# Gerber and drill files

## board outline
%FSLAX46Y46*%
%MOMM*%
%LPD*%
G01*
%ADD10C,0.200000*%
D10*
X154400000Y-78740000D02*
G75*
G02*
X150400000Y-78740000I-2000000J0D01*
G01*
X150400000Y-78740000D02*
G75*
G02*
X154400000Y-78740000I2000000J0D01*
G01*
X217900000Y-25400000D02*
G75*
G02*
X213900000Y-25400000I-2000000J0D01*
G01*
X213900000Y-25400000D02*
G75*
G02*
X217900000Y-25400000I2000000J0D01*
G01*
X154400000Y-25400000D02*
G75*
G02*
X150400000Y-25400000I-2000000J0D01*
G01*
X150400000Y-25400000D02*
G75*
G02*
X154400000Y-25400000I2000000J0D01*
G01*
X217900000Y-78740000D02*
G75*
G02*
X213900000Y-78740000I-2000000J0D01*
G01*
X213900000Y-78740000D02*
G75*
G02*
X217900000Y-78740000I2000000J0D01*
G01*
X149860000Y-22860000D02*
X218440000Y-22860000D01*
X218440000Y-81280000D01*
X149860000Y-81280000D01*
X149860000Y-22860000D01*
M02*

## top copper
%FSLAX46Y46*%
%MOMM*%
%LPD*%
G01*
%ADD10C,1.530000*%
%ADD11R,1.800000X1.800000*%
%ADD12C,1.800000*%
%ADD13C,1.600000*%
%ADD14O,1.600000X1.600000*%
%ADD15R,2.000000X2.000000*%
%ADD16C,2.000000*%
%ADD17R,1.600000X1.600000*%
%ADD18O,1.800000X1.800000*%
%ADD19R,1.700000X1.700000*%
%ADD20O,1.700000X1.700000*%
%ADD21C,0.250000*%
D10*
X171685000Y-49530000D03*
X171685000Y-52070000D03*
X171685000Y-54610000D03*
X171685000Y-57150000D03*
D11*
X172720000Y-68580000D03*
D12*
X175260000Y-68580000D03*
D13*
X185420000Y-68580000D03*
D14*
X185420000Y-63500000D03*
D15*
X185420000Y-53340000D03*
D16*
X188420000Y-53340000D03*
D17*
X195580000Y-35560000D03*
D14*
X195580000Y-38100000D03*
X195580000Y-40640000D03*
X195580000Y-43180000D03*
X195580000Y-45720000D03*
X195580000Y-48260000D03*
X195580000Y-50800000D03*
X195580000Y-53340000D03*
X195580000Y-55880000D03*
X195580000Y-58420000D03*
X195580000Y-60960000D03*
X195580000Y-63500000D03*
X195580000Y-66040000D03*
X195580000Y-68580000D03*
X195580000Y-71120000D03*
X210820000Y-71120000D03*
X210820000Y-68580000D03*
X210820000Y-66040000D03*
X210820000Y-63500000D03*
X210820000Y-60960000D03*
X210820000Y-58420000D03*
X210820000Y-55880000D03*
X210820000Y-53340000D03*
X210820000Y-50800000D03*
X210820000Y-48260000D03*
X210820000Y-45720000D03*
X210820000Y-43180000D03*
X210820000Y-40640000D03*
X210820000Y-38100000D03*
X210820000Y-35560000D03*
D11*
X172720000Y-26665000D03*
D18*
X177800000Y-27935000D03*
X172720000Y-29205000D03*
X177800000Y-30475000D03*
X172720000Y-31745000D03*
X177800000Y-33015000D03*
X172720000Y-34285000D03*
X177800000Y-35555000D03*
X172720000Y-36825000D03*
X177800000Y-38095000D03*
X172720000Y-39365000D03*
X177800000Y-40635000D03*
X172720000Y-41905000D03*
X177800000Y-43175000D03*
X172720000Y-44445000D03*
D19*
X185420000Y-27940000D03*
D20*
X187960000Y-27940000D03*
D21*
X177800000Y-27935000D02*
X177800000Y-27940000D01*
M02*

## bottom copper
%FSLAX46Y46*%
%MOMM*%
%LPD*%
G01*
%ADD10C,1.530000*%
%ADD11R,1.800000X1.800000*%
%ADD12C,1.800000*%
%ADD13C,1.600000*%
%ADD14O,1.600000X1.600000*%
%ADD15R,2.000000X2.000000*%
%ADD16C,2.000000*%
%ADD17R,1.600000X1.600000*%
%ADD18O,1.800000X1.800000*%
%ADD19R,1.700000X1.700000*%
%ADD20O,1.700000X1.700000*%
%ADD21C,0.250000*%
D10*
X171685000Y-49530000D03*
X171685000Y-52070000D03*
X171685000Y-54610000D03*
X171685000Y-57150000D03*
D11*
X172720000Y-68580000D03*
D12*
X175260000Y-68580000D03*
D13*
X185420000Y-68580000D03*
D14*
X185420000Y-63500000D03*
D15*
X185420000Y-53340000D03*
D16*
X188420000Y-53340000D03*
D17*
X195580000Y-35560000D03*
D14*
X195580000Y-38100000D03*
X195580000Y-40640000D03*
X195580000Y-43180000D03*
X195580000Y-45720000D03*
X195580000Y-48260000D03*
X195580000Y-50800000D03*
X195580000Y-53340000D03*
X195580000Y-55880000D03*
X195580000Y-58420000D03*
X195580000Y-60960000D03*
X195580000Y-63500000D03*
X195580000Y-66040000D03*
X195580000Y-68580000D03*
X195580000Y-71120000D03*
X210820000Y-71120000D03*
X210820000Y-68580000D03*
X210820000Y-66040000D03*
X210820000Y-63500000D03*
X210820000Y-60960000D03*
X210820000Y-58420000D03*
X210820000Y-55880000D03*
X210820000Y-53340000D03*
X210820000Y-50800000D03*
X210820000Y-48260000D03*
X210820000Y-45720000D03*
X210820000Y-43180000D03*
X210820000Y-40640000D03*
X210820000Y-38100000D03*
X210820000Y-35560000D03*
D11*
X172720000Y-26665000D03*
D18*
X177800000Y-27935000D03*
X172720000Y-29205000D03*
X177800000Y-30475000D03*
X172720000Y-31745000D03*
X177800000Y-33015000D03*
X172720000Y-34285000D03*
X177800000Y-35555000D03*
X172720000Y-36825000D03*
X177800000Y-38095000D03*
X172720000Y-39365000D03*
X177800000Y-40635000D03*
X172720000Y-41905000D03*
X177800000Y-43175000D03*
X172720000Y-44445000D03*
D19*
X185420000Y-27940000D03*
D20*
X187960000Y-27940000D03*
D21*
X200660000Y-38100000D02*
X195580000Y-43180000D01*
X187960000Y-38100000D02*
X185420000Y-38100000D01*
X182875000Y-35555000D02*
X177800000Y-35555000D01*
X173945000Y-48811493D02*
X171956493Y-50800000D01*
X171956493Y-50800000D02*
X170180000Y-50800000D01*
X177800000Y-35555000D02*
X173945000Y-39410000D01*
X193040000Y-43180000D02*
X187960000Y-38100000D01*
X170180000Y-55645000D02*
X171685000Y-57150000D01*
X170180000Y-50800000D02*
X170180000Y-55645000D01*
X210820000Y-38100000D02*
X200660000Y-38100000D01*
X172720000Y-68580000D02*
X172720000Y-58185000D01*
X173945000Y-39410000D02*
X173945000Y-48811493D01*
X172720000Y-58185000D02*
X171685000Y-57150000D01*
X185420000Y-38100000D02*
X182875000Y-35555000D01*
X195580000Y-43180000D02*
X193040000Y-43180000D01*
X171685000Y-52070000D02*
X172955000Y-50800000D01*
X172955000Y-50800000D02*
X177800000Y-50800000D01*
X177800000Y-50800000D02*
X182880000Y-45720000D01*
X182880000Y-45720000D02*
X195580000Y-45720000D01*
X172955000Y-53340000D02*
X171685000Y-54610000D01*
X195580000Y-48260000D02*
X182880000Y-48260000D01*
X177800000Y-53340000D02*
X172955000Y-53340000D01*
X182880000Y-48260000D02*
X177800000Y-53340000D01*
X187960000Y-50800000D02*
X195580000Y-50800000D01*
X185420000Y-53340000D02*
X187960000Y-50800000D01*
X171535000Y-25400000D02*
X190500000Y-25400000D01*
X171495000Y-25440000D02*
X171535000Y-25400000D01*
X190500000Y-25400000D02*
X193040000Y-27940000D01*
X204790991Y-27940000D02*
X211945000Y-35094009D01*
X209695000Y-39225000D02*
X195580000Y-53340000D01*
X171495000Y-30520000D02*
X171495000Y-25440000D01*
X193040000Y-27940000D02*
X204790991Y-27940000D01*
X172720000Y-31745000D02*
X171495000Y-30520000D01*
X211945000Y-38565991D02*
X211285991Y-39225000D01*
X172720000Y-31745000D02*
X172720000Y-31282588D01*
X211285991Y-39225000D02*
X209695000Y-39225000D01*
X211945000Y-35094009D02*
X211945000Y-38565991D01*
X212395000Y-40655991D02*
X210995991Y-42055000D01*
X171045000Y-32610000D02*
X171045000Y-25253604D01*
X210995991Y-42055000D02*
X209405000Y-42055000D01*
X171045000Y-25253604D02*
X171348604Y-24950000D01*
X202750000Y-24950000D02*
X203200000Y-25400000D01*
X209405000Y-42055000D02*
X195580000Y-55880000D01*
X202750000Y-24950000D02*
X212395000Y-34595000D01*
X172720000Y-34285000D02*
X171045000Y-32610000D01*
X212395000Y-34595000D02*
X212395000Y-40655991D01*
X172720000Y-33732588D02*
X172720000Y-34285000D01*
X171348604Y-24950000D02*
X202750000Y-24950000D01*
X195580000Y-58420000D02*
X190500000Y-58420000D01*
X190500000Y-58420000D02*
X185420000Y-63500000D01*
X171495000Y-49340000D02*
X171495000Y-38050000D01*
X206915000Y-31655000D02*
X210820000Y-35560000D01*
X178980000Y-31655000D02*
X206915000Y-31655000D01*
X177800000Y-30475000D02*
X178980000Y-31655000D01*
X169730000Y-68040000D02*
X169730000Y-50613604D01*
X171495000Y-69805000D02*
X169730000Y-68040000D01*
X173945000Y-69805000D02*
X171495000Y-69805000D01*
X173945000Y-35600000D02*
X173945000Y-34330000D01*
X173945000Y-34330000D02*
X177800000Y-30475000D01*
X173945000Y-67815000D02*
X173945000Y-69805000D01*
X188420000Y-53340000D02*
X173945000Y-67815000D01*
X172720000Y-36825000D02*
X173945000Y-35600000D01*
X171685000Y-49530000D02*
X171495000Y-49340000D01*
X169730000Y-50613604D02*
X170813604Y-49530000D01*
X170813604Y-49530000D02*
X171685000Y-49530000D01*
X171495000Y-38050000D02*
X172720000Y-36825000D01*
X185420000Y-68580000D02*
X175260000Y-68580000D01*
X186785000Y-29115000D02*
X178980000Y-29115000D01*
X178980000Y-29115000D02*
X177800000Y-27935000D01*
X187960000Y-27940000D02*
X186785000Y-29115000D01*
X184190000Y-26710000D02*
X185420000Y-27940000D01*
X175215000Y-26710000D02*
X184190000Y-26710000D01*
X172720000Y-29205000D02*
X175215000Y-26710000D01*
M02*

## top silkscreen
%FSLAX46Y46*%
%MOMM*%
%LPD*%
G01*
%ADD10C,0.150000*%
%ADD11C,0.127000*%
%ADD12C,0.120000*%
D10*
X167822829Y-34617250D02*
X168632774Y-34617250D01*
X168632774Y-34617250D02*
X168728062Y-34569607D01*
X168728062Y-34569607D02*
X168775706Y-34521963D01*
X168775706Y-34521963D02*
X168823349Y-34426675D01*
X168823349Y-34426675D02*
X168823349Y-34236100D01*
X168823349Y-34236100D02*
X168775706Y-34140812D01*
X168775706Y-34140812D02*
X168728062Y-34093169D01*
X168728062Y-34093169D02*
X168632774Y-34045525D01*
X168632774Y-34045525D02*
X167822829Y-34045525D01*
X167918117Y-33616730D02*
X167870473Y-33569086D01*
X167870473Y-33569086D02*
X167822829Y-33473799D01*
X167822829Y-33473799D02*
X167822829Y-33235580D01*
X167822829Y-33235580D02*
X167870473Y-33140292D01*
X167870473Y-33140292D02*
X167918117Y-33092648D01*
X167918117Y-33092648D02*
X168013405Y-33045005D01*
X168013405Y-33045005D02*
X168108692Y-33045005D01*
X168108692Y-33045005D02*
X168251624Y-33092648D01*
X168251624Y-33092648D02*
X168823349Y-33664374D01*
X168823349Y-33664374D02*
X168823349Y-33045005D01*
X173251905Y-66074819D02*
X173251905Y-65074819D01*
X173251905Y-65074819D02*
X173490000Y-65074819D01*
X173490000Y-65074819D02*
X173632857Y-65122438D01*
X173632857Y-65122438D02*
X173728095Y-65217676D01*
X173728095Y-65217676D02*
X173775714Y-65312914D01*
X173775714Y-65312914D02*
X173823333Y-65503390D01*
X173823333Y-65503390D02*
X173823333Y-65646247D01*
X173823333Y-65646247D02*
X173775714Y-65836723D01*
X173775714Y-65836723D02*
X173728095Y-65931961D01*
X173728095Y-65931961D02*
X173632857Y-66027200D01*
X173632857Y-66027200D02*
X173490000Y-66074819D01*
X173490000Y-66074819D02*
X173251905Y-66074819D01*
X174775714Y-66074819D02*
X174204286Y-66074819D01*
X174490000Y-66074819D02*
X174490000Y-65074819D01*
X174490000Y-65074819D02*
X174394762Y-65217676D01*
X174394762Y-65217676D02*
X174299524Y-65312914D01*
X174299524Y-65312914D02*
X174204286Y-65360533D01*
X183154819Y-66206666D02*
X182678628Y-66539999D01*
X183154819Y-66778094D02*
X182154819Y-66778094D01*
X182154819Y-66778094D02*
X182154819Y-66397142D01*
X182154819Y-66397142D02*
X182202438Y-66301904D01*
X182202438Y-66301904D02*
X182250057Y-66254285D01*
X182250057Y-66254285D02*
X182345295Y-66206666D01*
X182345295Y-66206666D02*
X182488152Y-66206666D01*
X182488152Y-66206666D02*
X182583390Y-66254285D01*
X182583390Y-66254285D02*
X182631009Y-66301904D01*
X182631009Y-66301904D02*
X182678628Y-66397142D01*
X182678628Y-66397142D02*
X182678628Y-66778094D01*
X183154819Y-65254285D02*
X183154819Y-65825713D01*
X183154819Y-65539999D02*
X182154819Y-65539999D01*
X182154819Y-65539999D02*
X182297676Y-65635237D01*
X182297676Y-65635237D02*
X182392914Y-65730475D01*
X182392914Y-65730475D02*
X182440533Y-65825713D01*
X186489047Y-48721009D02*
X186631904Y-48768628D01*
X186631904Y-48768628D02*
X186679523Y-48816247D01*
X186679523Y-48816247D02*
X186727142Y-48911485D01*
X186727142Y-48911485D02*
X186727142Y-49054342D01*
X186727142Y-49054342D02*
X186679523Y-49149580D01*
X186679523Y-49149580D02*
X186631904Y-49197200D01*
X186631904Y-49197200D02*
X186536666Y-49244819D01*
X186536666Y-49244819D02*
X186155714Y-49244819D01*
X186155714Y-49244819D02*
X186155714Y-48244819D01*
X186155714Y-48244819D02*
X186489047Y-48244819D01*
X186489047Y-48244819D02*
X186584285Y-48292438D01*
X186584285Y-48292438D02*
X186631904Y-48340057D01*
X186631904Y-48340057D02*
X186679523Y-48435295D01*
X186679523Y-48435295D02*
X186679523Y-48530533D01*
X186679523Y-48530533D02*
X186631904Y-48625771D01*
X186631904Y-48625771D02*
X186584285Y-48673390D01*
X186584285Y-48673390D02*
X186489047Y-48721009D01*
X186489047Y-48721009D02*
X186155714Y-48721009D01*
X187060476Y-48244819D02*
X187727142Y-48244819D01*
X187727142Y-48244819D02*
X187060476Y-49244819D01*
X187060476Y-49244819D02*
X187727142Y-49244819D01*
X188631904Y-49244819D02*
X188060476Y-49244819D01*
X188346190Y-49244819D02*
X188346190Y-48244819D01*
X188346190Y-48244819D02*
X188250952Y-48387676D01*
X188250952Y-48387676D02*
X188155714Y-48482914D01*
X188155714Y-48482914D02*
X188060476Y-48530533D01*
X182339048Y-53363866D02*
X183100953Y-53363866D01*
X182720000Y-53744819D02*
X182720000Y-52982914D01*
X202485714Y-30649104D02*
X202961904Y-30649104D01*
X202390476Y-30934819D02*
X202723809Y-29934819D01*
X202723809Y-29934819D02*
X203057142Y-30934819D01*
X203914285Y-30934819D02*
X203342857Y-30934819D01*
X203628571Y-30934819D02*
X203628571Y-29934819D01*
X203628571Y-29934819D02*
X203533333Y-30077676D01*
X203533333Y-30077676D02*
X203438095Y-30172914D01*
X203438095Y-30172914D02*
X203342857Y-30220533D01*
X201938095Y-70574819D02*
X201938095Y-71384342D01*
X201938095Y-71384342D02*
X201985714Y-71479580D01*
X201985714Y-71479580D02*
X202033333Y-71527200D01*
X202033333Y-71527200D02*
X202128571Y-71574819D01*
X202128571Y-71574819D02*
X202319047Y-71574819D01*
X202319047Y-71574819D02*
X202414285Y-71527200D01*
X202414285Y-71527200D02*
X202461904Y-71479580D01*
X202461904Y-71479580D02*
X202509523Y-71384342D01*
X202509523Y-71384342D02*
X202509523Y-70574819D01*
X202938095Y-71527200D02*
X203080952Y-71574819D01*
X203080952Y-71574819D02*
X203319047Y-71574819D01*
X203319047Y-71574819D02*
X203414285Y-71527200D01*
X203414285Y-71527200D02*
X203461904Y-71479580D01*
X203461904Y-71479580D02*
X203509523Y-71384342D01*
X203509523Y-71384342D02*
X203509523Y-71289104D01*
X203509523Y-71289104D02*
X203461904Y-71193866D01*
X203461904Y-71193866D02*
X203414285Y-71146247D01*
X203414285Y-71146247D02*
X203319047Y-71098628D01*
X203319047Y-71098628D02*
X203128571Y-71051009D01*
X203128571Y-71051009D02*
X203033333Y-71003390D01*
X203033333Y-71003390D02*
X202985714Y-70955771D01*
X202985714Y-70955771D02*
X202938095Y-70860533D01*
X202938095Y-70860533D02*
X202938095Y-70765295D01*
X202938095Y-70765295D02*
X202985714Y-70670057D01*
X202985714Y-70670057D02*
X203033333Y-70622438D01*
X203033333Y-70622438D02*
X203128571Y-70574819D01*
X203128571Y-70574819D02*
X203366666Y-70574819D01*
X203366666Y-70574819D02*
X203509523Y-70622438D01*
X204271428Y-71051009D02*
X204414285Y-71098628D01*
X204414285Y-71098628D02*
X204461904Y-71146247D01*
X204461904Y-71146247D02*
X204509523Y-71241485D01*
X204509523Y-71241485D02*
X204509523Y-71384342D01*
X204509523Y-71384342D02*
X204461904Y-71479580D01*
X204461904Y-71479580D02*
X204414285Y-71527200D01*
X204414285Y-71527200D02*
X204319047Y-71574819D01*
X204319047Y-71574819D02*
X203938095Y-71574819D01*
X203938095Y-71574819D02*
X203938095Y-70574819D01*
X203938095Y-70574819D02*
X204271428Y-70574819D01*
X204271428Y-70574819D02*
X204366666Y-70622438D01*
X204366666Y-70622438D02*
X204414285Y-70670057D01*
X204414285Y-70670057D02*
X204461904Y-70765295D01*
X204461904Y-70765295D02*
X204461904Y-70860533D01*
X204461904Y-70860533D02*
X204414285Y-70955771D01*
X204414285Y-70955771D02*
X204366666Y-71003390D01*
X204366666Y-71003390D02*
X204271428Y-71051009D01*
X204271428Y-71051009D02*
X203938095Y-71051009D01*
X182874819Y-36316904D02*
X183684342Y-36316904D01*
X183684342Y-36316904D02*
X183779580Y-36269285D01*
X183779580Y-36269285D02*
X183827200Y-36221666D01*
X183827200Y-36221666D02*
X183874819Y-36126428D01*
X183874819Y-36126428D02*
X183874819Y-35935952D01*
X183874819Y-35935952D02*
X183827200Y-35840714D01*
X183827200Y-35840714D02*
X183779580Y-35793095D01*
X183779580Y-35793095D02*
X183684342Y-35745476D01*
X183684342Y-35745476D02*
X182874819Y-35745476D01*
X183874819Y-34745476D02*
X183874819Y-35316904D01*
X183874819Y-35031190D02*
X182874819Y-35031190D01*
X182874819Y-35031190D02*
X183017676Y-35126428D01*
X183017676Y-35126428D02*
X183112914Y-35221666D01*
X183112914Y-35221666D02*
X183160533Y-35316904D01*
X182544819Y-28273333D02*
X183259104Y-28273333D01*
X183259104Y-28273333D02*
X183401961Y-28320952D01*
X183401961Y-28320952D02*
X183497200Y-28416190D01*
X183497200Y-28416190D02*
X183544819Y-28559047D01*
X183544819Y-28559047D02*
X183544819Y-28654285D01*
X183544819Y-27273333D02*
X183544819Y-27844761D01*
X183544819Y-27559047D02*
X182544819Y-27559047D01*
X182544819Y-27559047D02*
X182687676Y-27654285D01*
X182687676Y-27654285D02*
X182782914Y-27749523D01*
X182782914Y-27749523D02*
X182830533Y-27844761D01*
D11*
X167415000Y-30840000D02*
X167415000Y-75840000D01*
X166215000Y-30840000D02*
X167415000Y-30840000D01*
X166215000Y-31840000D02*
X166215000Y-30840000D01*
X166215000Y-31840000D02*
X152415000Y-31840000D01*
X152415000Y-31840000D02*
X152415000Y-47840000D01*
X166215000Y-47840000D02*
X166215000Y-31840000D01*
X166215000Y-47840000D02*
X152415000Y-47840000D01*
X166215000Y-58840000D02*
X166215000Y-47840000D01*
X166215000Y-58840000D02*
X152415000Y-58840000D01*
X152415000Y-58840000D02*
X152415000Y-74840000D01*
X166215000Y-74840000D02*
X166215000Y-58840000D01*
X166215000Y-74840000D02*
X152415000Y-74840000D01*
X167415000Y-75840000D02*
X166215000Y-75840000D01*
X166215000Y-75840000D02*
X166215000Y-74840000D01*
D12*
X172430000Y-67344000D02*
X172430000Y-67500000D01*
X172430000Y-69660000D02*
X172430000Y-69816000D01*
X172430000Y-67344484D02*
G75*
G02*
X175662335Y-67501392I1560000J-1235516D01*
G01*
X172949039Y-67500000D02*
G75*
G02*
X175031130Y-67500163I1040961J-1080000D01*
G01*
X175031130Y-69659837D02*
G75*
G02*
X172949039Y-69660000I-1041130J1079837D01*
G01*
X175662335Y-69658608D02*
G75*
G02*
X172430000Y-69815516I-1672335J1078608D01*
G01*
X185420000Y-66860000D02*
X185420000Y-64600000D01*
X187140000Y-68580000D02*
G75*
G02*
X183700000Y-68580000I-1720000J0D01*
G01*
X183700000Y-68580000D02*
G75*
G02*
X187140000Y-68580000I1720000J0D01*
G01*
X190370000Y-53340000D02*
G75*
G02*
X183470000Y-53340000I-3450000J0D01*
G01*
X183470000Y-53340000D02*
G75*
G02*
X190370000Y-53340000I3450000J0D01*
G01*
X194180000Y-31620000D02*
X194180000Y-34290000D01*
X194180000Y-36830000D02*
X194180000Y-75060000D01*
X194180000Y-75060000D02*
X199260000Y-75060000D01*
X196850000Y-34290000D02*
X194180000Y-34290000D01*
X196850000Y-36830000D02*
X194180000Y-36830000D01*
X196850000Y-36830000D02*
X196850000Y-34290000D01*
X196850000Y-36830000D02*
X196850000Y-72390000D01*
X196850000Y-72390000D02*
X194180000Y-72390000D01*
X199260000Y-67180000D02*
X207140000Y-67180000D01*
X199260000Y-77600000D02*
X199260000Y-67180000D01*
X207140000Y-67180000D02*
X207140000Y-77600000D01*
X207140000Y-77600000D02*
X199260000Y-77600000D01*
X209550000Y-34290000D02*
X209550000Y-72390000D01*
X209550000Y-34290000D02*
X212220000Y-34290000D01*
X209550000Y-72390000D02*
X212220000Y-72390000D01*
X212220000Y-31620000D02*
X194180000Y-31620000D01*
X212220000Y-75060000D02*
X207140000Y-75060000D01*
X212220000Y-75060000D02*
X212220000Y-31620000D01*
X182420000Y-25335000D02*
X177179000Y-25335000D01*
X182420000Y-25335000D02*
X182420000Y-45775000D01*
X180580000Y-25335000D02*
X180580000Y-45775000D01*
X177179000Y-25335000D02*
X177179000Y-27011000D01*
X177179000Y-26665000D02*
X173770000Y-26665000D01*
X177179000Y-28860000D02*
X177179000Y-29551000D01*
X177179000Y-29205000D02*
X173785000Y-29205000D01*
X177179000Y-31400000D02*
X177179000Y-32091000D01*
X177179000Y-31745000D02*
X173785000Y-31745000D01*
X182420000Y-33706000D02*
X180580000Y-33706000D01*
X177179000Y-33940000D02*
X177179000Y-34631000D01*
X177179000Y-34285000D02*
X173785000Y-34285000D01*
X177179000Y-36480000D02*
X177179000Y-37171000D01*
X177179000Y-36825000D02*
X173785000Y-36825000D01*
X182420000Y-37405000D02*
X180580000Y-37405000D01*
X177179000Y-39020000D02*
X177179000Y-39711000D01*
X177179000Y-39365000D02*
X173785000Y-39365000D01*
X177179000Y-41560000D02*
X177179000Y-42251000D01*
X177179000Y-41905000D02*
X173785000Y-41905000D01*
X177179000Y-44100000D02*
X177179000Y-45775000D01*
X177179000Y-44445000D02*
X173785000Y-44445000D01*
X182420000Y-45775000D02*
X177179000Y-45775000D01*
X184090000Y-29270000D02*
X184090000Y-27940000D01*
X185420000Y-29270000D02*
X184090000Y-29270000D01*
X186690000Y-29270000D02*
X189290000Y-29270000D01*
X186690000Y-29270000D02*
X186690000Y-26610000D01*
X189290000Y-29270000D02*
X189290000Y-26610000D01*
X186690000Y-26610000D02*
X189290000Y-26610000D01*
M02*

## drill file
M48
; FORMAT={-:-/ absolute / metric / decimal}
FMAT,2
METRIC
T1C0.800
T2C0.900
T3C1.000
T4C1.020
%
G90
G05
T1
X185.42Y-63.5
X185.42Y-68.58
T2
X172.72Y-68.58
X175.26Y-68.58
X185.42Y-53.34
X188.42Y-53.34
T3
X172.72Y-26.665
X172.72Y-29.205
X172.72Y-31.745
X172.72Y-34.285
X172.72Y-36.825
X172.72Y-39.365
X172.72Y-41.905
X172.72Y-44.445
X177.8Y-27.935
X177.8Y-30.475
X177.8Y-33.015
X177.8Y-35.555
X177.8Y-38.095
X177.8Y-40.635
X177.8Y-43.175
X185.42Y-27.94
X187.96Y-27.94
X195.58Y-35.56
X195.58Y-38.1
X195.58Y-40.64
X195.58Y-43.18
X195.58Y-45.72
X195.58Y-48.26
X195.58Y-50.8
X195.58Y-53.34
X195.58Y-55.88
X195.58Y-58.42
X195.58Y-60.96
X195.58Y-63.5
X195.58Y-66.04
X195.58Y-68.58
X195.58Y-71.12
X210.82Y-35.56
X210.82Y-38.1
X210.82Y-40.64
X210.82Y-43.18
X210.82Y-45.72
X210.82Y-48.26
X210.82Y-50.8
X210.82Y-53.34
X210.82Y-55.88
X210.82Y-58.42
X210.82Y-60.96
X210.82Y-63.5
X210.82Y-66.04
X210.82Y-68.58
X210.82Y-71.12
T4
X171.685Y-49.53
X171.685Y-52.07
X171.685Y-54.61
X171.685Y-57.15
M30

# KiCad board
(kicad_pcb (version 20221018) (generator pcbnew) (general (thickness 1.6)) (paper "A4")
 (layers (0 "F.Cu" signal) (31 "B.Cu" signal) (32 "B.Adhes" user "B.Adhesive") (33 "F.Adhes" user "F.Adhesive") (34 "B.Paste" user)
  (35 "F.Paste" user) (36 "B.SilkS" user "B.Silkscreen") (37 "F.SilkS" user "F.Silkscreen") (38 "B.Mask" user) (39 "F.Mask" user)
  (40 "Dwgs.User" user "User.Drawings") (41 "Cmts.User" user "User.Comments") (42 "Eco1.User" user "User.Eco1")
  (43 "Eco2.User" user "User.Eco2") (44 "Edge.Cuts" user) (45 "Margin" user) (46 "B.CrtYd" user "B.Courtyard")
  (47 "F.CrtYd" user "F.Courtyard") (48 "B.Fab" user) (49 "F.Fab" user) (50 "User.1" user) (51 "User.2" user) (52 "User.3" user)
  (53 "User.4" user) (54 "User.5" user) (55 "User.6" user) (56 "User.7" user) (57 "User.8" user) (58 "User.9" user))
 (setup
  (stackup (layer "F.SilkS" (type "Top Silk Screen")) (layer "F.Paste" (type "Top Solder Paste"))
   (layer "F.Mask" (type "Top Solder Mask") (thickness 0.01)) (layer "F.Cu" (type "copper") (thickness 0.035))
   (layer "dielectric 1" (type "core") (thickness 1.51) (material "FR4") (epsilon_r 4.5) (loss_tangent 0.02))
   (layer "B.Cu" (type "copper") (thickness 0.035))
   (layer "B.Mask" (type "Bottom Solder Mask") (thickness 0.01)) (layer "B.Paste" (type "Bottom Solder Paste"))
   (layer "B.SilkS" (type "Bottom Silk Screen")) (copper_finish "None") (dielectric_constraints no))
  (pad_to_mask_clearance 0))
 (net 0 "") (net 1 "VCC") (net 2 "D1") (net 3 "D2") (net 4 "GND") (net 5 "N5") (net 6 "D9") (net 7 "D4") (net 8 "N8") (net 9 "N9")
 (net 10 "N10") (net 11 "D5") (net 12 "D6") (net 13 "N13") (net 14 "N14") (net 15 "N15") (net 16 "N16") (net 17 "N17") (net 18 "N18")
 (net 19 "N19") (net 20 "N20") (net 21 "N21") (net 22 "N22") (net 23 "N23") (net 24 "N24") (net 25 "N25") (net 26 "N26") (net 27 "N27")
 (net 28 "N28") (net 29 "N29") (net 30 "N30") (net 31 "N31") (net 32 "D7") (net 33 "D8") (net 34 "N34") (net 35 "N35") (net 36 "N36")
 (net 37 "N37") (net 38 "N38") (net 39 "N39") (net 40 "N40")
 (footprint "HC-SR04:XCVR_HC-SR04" (layer "F.Cu") (at 171.685 53.34 -90)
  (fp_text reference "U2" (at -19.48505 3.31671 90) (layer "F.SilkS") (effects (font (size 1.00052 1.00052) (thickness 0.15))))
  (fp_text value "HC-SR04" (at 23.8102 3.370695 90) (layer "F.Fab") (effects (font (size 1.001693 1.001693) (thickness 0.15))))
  (fp_line (start -22.5 4.27) (end 22.5 4.27) (stroke (width 0.127) (type solid)) (layer "F.SilkS"))
  (fp_line (start -22.5 5.47) (end -22.5 4.27) (stroke (width 0.127) (type solid)) (layer "F.SilkS"))
  (fp_line (start -21.5 5.47) (end -22.5 5.47) (stroke (width 0.127) (type solid)) (layer "F.SilkS"))
  (fp_line (start -21.5 5.47) (end -21.5 19.27) (stroke (width 0.127) (type solid)) (layer "F.SilkS"))
  (fp_line (start -21.5 19.27) (end -5.5 19.27) (stroke (width 0.127) (type solid)) (layer "F.SilkS"))
  (fp_line (start -5.5 5.47) (end -21.5 5.47) (stroke (width 0.127) (type solid)) (layer "F.SilkS"))
  (fp_line (start -5.5 5.47) (end -5.5 19.27) (stroke (width 0.127) (type solid)) (layer "F.SilkS"))
  (fp_line (start 5.5 5.47) (end -5.5 5.47) (stroke (width 0.127) (type solid)) (layer "F.SilkS"))
  (fp_line (start 5.5 5.47) (end 5.5 19.27) (stroke (width 0.127) (type solid)) (layer "F.SilkS"))
  (fp_line (start 5.5 19.27) (end 21.5 19.27) (stroke (width 0.127) (type solid)) (layer "F.SilkS"))
  (fp_line (start 21.5 5.47) (end 5.5 5.47) (stroke (width 0.127) (type solid)) (layer "F.SilkS"))
  (fp_line (start 21.5 5.47) (end 21.5 19.27) (stroke (width 0.127) (type solid)) (layer "F.SilkS"))
  (fp_line (start 22.5 4.27) (end 22.5 5.47) (stroke (width 0.127) (type solid)) (layer "F.SilkS"))
  (fp_line (start 22.5 5.47) (end 21.5 5.47) (stroke (width 0.127) (type solid)) (layer "F.SilkS"))
  (pad "1" thru_hole circle (at -3.81 0 270) (size 1.53 1.53) (drill 1.02) (layers "*.Cu" "*.Mask") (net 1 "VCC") (solder_mask_margin 0.102))
  (pad "2" thru_hole circle (at -1.27 0 270) (size 1.53 1.53) (drill 1.02) (layers "*.Cu" "*.Mask") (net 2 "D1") (solder_mask_margin 0.102))
  (pad "3" thru_hole circle (at 1.27 0 270) (size 1.53 1.53) (drill 1.02) (layers "*.Cu" "*.Mask") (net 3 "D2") (solder_mask_margin 0.102))
  (pad "4" thru_hole circle (at 3.81 0 270) (size 1.53 1.53) (drill 1.02) (layers "*.Cu" "*.Mask") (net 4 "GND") (solder_mask_margin 0.102)))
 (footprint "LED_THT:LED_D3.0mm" (layer "F.Cu") (at 172.72 68.58)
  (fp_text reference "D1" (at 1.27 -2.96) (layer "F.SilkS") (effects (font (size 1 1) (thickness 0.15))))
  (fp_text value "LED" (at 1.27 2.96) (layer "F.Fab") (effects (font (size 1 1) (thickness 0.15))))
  (fp_line (start -0.29 -1.236) (end -0.29 -1.08) (stroke (width 0.12) (type solid)) (layer "F.SilkS"))
  (fp_line (start -0.29 1.08) (end -0.29 1.236) (stroke (width 0.12) (type solid)) (layer "F.SilkS"))
  (fp_arc (start -0.29 -1.235516) (mid 1.366487 -1.987659) (end 2.942335 -1.078608) (stroke (width 0.12) (type solid)) (layer "F.SilkS"))
  (fp_arc (start 0.229039 -1.08) (mid 1.270117 -1.5) (end 2.31113 -1.079837) (stroke (width 0.12) (type solid)) (layer "F.SilkS"))
  (fp_arc (start 2.31113 1.079837) (mid 1.270117 1.5) (end 0.229039 1.08) (stroke (width 0.12) (type solid)) (layer "F.SilkS"))
  (fp_arc (start 2.942335 1.078608) (mid 1.366487 1.987659) (end -0.29 1.235516) (stroke (width 0.12) (type solid)) (layer "F.SilkS"))
  (pad "1" thru_hole rect (at 0 0) (size 1.8 1.8) (drill 0.9) (layers "*.Cu" "*.Mask") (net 4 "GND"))
  (pad "2" thru_hole circle (at 2.54 0) (size 1.8 1.8) (drill 0.9) (layers "*.Cu" "*.Mask") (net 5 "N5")))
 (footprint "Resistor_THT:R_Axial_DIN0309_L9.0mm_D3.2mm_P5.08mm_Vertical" (layer "F.Cu") (at 185.42 68.58 90)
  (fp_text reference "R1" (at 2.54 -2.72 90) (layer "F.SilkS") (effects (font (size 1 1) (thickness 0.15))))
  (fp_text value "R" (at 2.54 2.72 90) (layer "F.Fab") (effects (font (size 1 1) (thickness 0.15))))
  (fp_line (start 1.72 0) (end 3.98 0) (stroke (width 0.12) (type solid)) (layer "F.SilkS"))
  (fp_circle (center 0 0) (end 1.72 0) (stroke (width 0.12) (type solid)) (fill none) (layer "F.SilkS"))
  (pad "1" thru_hole circle (at 0 0 90) (size 1.6 1.6) (drill 0.8) (layers "*.Cu" "*.Mask") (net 5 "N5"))
  (pad "2" thru_hole oval (at 5.08 0 90) (size 1.6 1.6) (drill 0.8) (layers "*.Cu" "*.Mask") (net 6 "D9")))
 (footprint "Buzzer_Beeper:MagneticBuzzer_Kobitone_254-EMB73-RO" (layer "F.Cu") (at 185.42 53.34)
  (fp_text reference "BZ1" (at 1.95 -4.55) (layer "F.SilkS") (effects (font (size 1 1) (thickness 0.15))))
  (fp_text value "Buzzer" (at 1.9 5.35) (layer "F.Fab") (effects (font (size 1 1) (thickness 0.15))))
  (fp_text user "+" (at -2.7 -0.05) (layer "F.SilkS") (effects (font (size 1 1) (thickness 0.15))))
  (fp_circle (center 1.5 0) (end 4.95 0) (stroke (width 0.12) (type solid)) (fill none) (layer "F.SilkS"))
  (pad "1" thru_hole rect (at 0 0) (size 2 2) (drill 0.9) (layers "*.Cu" "*.Mask") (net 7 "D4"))
  (pad "2" thru_hole circle (at 3 0) (size 2 2) (drill 0.9) (layers "*.Cu" "*.Mask") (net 1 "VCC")))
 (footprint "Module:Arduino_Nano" (layer "F.Cu") (at 195.58 35.56)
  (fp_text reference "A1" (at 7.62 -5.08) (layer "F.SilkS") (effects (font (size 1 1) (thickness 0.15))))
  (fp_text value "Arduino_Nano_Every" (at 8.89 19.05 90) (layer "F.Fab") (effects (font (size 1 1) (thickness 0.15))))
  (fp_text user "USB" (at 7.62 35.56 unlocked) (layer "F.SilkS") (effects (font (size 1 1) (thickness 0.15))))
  (fp_line (start -1.4 -3.94) (end -1.4 -1.27) (stroke (width 0.12) (type solid)) (layer "F.SilkS"))
  (fp_line (start -1.4 1.27) (end -1.4 39.5) (stroke (width 0.12) (type solid)) (layer "F.SilkS"))
  (fp_line (start -1.4 39.5) (end 3.68 39.5) (stroke (width 0.12) (type solid)) (layer "F.SilkS"))
  (fp_line (start 1.27 -1.27) (end -1.4 -1.27) (stroke (width 0.12) (type solid)) (layer "F.SilkS"))
  (fp_line (start 1.27 1.27) (end -1.4 1.27) (stroke (width 0.12) (type solid)) (layer "F.SilkS"))
  (fp_line (start 1.27 1.27) (end 1.27 -1.27) (stroke (width 0.12) (type solid)) (layer "F.SilkS"))
  (fp_line (start 1.27 1.27) (end 1.27 36.83) (stroke (width 0.12) (type solid)) (layer "F.SilkS"))
  (fp_line (start 1.27 36.83) (end -1.4 36.83) (stroke (width 0.12) (type solid)) (layer "F.SilkS"))
  (fp_line (start 3.68 31.62) (end 11.56 31.62) (stroke (width 0.12) (type solid)) (layer "F.SilkS"))
  (fp_line (start 3.68 42.04) (end 3.68 31.62) (stroke (width 0.12) (type solid)) (layer "F.SilkS"))
  (fp_line (start 11.56 31.62) (end 11.56 42.04) (stroke (width 0.12) (type solid)) (layer "F.SilkS"))
  (fp_line (start 11.56 42.04) (end 3.68 42.04) (stroke (width 0.12) (type solid)) (layer "F.SilkS"))
  (fp_line (start 13.97 -1.27) (end 13.97 36.83) (stroke (width 0.12) (type solid)) (layer "F.SilkS"))
  (fp_line (start 13.97 -1.27) (end 16.64 -1.27) (stroke (width 0.12) (type solid)) (layer "F.SilkS"))
  (fp_line (start 13.97 36.83) (end 16.64 36.83) (stroke (width 0.12) (type solid)) (layer "F.SilkS"))
  (fp_line (start 16.64 -3.94) (end -1.4 -3.94) (stroke (width 0.12) (type solid)) (layer "F.SilkS"))
  (fp_line (start 16.64 39.5) (end 11.56 39.5) (stroke (width 0.12) (type solid)) (layer "F.SilkS"))
  (fp_line (start 16.64 39.5) (end 16.64 -3.94) (stroke (width 0.12) (type solid)) (layer "F.SilkS"))
  (pad "1" thru_hole rect (at 0 0) (size 1.6 1.6) (drill 1) (layers "*.Cu" "*.Mask") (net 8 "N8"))
  (pad "2" thru_hole oval (at 0 2.54) (size 1.6 1.6) (drill 1) (layers "*.Cu" "*.Mask") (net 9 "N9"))
  (pad "3" thru_hole oval (at 0 5.08) (size 1.6 1.6) (drill 1) (layers "*.Cu" "*.Mask") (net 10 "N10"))
  (pad "4" thru_hole oval (at 0 7.62) (size 1.6 1.6) (drill 1) (layers "*.Cu" "*.Mask") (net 4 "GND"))
  (pad "5" thru_hole oval (at 0 10.16) (size 1.6 1.6) (drill 1) (layers "*.Cu" "*.Mask") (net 2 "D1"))
  (pad "6" thru_hole oval (at 0 12.7) (size 1.6 1.6) (drill 1) (layers "*.Cu" "*.Mask") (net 3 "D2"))
  (pad "7" thru_hole oval (at 0 15.24) (size 1.6 1.6) (drill 1) (layers "*.Cu" "*.Mask") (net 7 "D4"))
  (pad "8" thru_hole oval (at 0 17.78) (size 1.6 1.6) (drill 1) (layers "*.Cu" "*.Mask") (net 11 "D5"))
  (pad "9" thru_hole oval (at 0 20.32) (size 1.6 1.6) (drill 1) (layers "*.Cu" "*.Mask") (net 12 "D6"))
  (pad "10" thru_hole oval (at 0 22.86) (size 1.6 1.6) (drill 1) (layers "*.Cu" "*.Mask") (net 6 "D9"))
  (pad "11" thru_hole oval (at 0 25.4) (size 1.6 1.6) (drill 1) (layers "*.Cu" "*.Mask") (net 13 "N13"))
  (pad "12" thru_hole oval (at 0 27.94) (size 1.6 1.6) (drill 1) (layers "*.Cu" "*.Mask") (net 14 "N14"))
  (pad "13" thru_hole oval (at 0 30.48) (size 1.6 1.6) (drill 1) (layers "*.Cu" "*.Mask") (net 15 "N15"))
  (pad "14" thru_hole oval (at 0 33.02) (size 1.6 1.6) (drill 1) (layers "*.Cu" "*.Mask") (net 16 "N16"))
  (pad "15" thru_hole oval (at 0 35.56) (size 1.6 1.6) (drill 1) (layers "*.Cu" "*.Mask") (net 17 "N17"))
  (pad "16" thru_hole oval (at 15.24 35.56) (size 1.6 1.6) (drill 1) (layers "*.Cu" "*.Mask") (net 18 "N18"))
  (pad "17" thru_hole oval (at 15.24 33.02) (size 1.6 1.6) (drill 1) (layers "*.Cu" "*.Mask") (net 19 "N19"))
  (pad "18" thru_hole oval (at 15.24 30.48) (size 1.6 1.6) (drill 1) (layers "*.Cu" "*.Mask") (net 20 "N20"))
  (pad "19" thru_hole oval (at 15.24 27.94) (size 1.6 1.6) (drill 1) (layers "*.Cu" "*.Mask") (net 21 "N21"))
  (pad "20" thru_hole oval (at 15.24 25.4) (size 1.6 1.6) (drill 1) (layers "*.Cu" "*.Mask") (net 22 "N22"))
  (pad "21" thru_hole oval (at 15.24 22.86) (size 1.6 1.6) (drill 1) (layers "*.Cu" "*.Mask") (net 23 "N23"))
  (pad "22" thru_hole oval (at 15.24 20.32) (size 1.6 1.6) (drill 1) (layers "*.Cu" "*.Mask") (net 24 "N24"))
  (pad "23" thru_hole oval (at 15.24 17.78) (size 1.6 1.6) (drill 1) (layers "*.Cu" "*.Mask") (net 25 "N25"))
  (pad "24" thru_hole oval (at 15.24 15.24) (size 1.6 1.6) (drill 1) (layers "*.Cu" "*.Mask") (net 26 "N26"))
  (pad "25" thru_hole oval (at 15.24 12.7) (size 1.6 1.6) (drill 1) (layers "*.Cu" "*.Mask") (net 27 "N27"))
  (pad "26" thru_hole oval (at 15.24 10.16) (size 1.6 1.6) (drill 1) (layers "*.Cu" "*.Mask") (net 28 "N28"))
  (pad "27" thru_hole oval (at 15.24 7.62) (size 1.6 1.6) (drill 1) (layers "*.Cu" "*.Mask") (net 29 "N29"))
  (pad "28" thru_hole oval (at 15.24 5.08) (size 1.6 1.6) (drill 1) (layers "*.Cu" "*.Mask") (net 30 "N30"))
  (pad "29" thru_hole oval (at 15.24 2.54) (size 1.6 1.6) (drill 1) (layers "*.Cu" "*.Mask") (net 4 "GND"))
  (pad "30" thru_hole oval (at 15.24 0) (size 1.6 1.6) (drill 1) (layers "*.Cu" "*.Mask") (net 1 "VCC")))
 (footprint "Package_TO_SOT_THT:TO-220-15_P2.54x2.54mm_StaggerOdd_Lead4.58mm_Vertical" (layer "F.Cu") (at 172.72 26.665 -90)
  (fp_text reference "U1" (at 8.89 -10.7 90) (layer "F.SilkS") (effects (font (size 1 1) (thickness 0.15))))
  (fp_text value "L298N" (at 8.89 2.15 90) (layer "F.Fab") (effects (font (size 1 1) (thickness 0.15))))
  (fp_line (start -1.33 -9.7) (end -1.33 -4.459) (stroke (width 0.12) (type solid)) (layer "F.SilkS"))
  (fp_line (start -1.33 -9.7) (end 19.11 -9.7) (stroke (width 0.12) (type solid)) (layer "F.SilkS"))
  (fp_line (start -1.33 -7.86) (end 19.11 -7.86) (stroke (width 0.12) (type solid)) (layer "F.SilkS"))
  (fp_line (start -1.33 -4.459) (end 0.346 -4.459) (stroke (width 0.12) (type solid)) (layer "F.SilkS"))
  (fp_line (start 0 -4.459) (end 0 -1.05) (stroke (width 0.12) (type solid)) (layer "F.SilkS"))
  (fp_line (start 2.195 -4.459) (end 2.886 -4.459) (stroke (width 0.12) (type solid)) (layer "F.SilkS"))
  (fp_line (start 2.54 -4.459) (end 2.54 -1.065) (stroke (width 0.12) (type solid)) (layer "F.SilkS"))
  (fp_line (start 4.735 -4.459) (end 5.426 -4.459) (stroke (width 0.12) (type solid)) (layer "F.SilkS"))
  (fp_line (start 5.08 -4.459) (end 5.08 -1.065) (stroke (width 0.12) (type solid)) (layer "F.SilkS"))
  (fp_line (start 7.041 -9.7) (end 7.041 -7.86) (stroke (width 0.12) (type solid)) (layer "F.SilkS"))
  (fp_line (start 7.275 -4.459) (end 7.966 -4.459) (stroke (width 0.12) (type solid)) (layer "F.SilkS"))
  (fp_line (start 7.62 -4.459) (end 7.62 -1.065) (stroke (width 0.12) (type solid)) (layer "F.SilkS"))
  (fp_line (start 9.815 -4.459) (end 10.506 -4.459) (stroke (width 0.12) (type solid)) (layer "F.SilkS"))
  (fp_line (start 10.16 -4.459) (end 10.16 -1.065) (stroke (width 0.12) (type solid)) (layer "F.SilkS"))
  (fp_line (start 10.74 -9.7) (end 10.74 -7.86) (stroke (width 0.12) (type solid)) (layer "F.SilkS"))
  (fp_line (start 12.355 -4.459) (end 13.046 -4.459) (stroke (width 0.12) (type solid)) (layer "F.SilkS"))
  (fp_line (start 12.7 -4.459) (end 12.7 -1.065) (stroke (width 0.12) (type solid)) (layer "F.SilkS"))
  (fp_line (start 14.895 -4.459) (end 15.586 -4.459) (stroke (width 0.12) (type solid)) (layer "F.SilkS"))
  (fp_line (start 15.24 -4.459) (end 15.24 -1.065) (stroke (width 0.12) (type solid)) (layer "F.SilkS"))
  (fp_line (start 17.435 -4.459) (end 19.11 -4.459) (stroke (width 0.12) (type solid)) (layer "F.SilkS"))
  (fp_line (start 17.78 -4.459) (end 17.78 -1.065) (stroke (width 0.12) (type solid)) (layer "F.SilkS"))
  (fp_line (start 19.11 -9.7) (end 19.11 -4.459) (stroke (width 0.12) (type solid)) (layer "F.SilkS"))
  (pad "1" thru_hole rect (at 0 0 270) (size 1.8 1.8) (drill 1) (layers "*.Cu" "*.Mask") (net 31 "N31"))
  (pad "2" thru_hole oval (at 1.27 -5.08 270) (size 1.8 1.8) (drill 1) (layers "*.Cu" "*.Mask") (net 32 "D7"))
  (pad "3" thru_hole oval (at 2.54 0 270) (size 1.8 1.8) (drill 1) (layers "*.Cu" "*.Mask") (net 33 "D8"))
  (pad "4" thru_hole oval (at 3.81 -5.08 270) (size 1.8 1.8) (drill 1) (layers "*.Cu" "*.Mask") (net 1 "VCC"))
  (pad "5" thru_hole oval (at 5.08 0 270) (size 1.8 1.8) (drill 1) (layers "*.Cu" "*.Mask") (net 11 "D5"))
  (pad "6" thru_hole oval (at 6.35 -5.08 270) (size 1.8 1.8) (drill 1) (layers "*.Cu" "*.Mask") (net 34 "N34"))
  (pad "7" thru_hole oval (at 7.62 0 270) (size 1.8 1.8) (drill 1) (layers "*.Cu" "*.Mask") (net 12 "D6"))
  (pad "8" thru_hole oval (at 8.89 -5.08 270) (size 1.8 1.8) (drill 1) (layers "*.Cu" "*.Mask") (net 4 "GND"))
  (pad "9" thru_hole oval (at 10.16 0 270) (size 1.8 1.8) (drill 1) (layers "*.Cu" "*.Mask") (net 1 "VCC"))
  (pad "10" thru_hole oval (at 11.43 -5.08 270) (size 1.8 1.8) (drill 1) (layers "*.Cu" "*.Mask") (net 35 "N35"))
  (pad "11" thru_hole oval (at 12.7 0 270) (size 1.8 1.8) (drill 1) (layers "*.Cu" "*.Mask") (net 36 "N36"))
  (pad "12" thru_hole oval (at 13.97 -5.08 270) (size 1.8 1.8) (drill 1) (layers "*.Cu" "*.Mask") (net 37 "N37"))
  (pad "13" thru_hole oval (at 15.24 0 270) (size 1.8 1.8) (drill 1) (layers "*.Cu" "*.Mask") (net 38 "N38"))
  (pad "14" thru_hole oval (at 16.51 -5.08 270) (size 1.8 1.8) (drill 1) (layers "*.Cu" "*.Mask") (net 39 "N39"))
  (pad "15" thru_hole oval (at 17.78 0 270) (size 1.8 1.8) (drill 1) (layers "*.Cu" "*.Mask") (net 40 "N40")))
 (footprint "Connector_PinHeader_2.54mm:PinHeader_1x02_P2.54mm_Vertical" (layer "F.Cu") (at 185.42 27.94 90)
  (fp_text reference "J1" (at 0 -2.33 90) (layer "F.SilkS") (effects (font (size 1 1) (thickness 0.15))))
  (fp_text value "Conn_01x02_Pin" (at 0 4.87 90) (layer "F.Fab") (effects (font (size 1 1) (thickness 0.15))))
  (fp_line (start -1.33 -1.33) (end 0 -1.33) (stroke (width 0.12) (type solid)) (layer "F.SilkS"))
  (fp_line (start -1.33 0) (end -1.33 -1.33) (stroke (width 0.12) (type solid)) (layer "F.SilkS"))
  (fp_line (start -1.33 1.27) (end -1.33 3.87) (stroke (width 0.12) (type solid)) (layer "F.SilkS"))
  (fp_line (start -1.33 1.27) (end 1.33 1.27) (stroke (width 0.12) (type solid)) (layer "F.SilkS"))
  (fp_line (start -1.33 3.87) (end 1.33 3.87) (stroke (width 0.12) (type solid)) (layer "F.SilkS"))
  (fp_line (start 1.33 1.27) (end 1.33 3.87) (stroke (width 0.12) (type solid)) (layer "F.SilkS"))
  (pad "1" thru_hole rect (at 0 0 90) (size 1.7 1.7) (drill 1) (layers "*.Cu" "*.Mask") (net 33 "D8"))
  (pad "2" thru_hole oval (at 0 2.54 90) (size 1.7 1.7) (drill 1) (layers "*.Cu" "*.Mask") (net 32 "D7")))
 (gr_circle (center 152.4 78.74) (end 154.4 78.74) (stroke (width 0.2) (type default)) (fill none) (layer "Edge.Cuts"))
 (gr_circle (center 215.9 25.4) (end 217.9 25.4) (stroke (width 0.2) (type default)) (fill none) (layer "Edge.Cuts"))
 (gr_circle (center 152.4 25.4) (end 154.4 25.4) (stroke (width 0.2) (type default)) (fill none) (layer "Edge.Cuts"))
 (gr_circle (center 215.9 78.74) (end 217.9 78.74) (stroke (width 0.2) (type default)) (fill none) (layer "Edge.Cuts"))
 (gr_rect (start 149.86 22.86) (end 218.44 81.28) (stroke (width 0.2) (type default)) (fill none) (layer "Edge.Cuts"))
 (segment (start 200.66 38.1) (end 195.58 43.18) (width 0.25) (layer "B.Cu") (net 4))
 (segment (start 187.96 38.1) (end 185.42 38.1) (width 0.25) (layer "B.Cu") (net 4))
 (segment (start 182.875 35.555) (end 177.8 35.555) (width 0.25) (layer "B.Cu") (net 4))
 (segment (start 173.945 48.811493) (end 171.956493 50.8) (width 0.25) (layer "B.Cu") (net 4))
 (segment (start 171.956493 50.8) (end 170.18 50.8) (width 0.25) (layer "B.Cu") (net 4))
 (segment (start 177.8 35.555) (end 173.945 39.41) (width 0.25) (layer "B.Cu") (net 4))
 (segment (start 193.04 43.18) (end 187.96 38.1) (width 0.25) (layer "B.Cu") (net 4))
 (segment (start 170.18 55.645) (end 171.685 57.15) (width 0.25) (layer "B.Cu") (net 4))
 (segment (start 170.18 50.8) (end 170.18 55.645) (width 0.25) (layer "B.Cu") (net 4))
 (segment (start 210.82 38.1) (end 200.66 38.1) (width 0.25) (layer "B.Cu") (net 4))
 (segment (start 172.72 68.58) (end 172.72 58.185) (width 0.25) (layer "B.Cu") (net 4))
 (segment (start 173.945 39.41) (end 173.945 48.811493) (width 0.25) (layer "B.Cu") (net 4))
 (segment (start 172.72 58.185) (end 171.685 57.15) (width 0.25) (layer "B.Cu") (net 4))
 (segment (start 185.42 38.1) (end 182.875 35.555) (width 0.25) (layer "B.Cu") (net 4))
 (segment (start 195.58 43.18) (end 193.04 43.18) (width 0.25) (layer "B.Cu") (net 4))
 (segment (start 171.685 52.07) (end 172.955 50.8) (width 0.25) (layer "B.Cu") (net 2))
 (segment (start 172.955 50.8) (end 177.8 50.8) (width 0.25) (layer "B.Cu") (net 2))
 (segment (start 177.8 50.8) (end 182.88 45.72) (width 0.25) (layer "B.Cu") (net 2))
 (segment (start 182.88 45.72) (end 195.58 45.72) (width 0.25) (layer "B.Cu") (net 2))
 (segment (start 172.955 53.34) (end 171.685 54.61) (width 0.25) (layer "B.Cu") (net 3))
 (segment (start 195.58 48.26) (end 182.88 48.26) (width 0.25) (layer "B.Cu") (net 3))
 (segment (start 177.8 53.34) (end 172.955 53.34) (width 0.25) (layer "B.Cu") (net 3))
 (segment (start 182.88 48.26) (end 177.8 53.34) (width 0.25) (layer "B.Cu") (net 3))
 (segment (start 187.96 50.8) (end 195.58 50.8) (width 0.25) (layer "B.Cu") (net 7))
 (segment (start 185.42 53.34) (end 187.96 50.8) (width 0.25) (layer "B.Cu") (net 7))
 (segment (start 171.535 25.4) (end 190.5 25.4) (width 0.25) (layer "B.Cu") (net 11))
 (segment (start 171.495 25.44) (end 171.535 25.4) (width 0.25) (layer "B.Cu") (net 11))
 (segment (start 190.5 25.4) (end 193.04 27.94) (width 0.25) (layer "B.Cu") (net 11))
 (segment (start 204.790991 27.94) (end 211.945 35.094009) (width 0.25) (layer "B.Cu") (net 11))
 (segment (start 209.695 39.225) (end 195.58 53.34) (width 0.25) (layer "B.Cu") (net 11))
 (segment (start 171.495 30.52) (end 171.495 25.44) (width 0.25) (layer "B.Cu") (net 11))
 (segment (start 193.04 27.94) (end 204.790991 27.94) (width 0.25) (layer "B.Cu") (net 11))
 (segment (start 172.72 31.745) (end 171.495 30.52) (width 0.25) (layer "B.Cu") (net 11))
 (segment (start 211.945 38.565991) (end 211.285991 39.225) (width 0.25) (layer "B.Cu") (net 11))
 (segment (start 172.72 31.745) (end 172.72 31.282588) (width 0.25) (layer "B.Cu") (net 11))
 (segment (start 211.285991 39.225) (end 209.695 39.225) (width 0.25) (layer "B.Cu") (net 11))
 (segment (start 211.945 35.094009) (end 211.945 38.565991) (width 0.25) (layer "B.Cu") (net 11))
 (segment (start 212.395 40.655991) (end 210.995991 42.055) (width 0.25) (layer "B.Cu") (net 12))
 (segment (start 171.045 32.61) (end 171.045 25.253604) (width 0.25) (layer "B.Cu") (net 12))
 (segment (start 210.995991 42.055) (end 209.405 42.055) (width 0.25) (layer "B.Cu") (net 12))
 (segment (start 171.045 25.253604) (end 171.348604 24.95) (width 0.25) (layer "B.Cu") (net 12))
 (segment (start 202.75 24.95) (end 203.2 25.4) (width 0.25) (layer "B.Cu") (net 12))
 (segment (start 209.405 42.055) (end 195.58 55.88) (width 0.25) (layer "B.Cu") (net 12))
 (segment (start 202.75 24.95) (end 212.395 34.595) (width 0.25) (layer "B.Cu") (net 12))
 (segment (start 172.72 34.285) (end 171.045 32.61) (width 0.25) (layer "B.Cu") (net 12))
 (segment (start 212.395 34.595) (end 212.395 40.655991) (width 0.25) (layer "B.Cu") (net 12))
 (segment (start 172.72 33.732588) (end 172.72 34.285) (width 0.25) (layer "B.Cu") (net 12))
 (segment (start 171.348604 24.95) (end 202.75 24.95) (width 0.25) (layer "B.Cu") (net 12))
 (segment (start 195.58 58.42) (end 190.5 58.42) (width 0.25) (layer "B.Cu") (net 6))
 (segment (start 190.5 58.42) (end 185.42 63.5) (width 0.25) (layer "B.Cu") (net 6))
 (segment (start 171.495 49.34) (end 171.495 38.05) (width 0.25) (layer "B.Cu") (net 1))
 (segment (start 206.915 31.655) (end 210.82 35.56) (width 0.25) (layer "B.Cu") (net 1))
 (segment (start 178.98 31.655) (end 206.915 31.655) (width 0.25) (layer "B.Cu") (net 1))
 (segment (start 177.8 30.475) (end 178.98 31.655) (width 0.25) (layer "B.Cu") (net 1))
 (segment (start 169.73 68.04) (end 169.73 50.613604) (width 0.25) (layer "B.Cu") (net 1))
 (segment (start 171.495 69.805) (end 169.73 68.04) (width 0.25) (layer "B.Cu") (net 1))
 (segment (start 173.945 69.805) (end 171.495 69.805) (width 0.25) (layer "B.Cu") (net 1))
 (segment (start 173.945 35.6) (end 173.945 34.33) (width 0.25) (layer "B.Cu") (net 1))
 (segment (start 173.945 34.33) (end 177.8 30.475) (width 0.25) (layer "B.Cu") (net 1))
 (segment (start 173.945 67.815) (end 173.945 69.805) (width 0.25) (layer "B.Cu") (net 1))
 (segment (start 188.42 53.34) (end 173.945 67.815) (width 0.25) (layer "B.Cu") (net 1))
 (segment (start 172.72 36.825) (end 173.945 35.6) (width 0.25) (layer "B.Cu") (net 1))
 (segment (start 171.685 49.53) (end 171.495 49.34) (width 0.25) (layer "B.Cu") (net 1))
 (segment (start 169.73 50.613604) (end 170.813604 49.53) (width 0.25) (layer "B.Cu") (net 1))
 (segment (start 170.813604 49.53) (end 171.685 49.53) (width 0.25) (layer "B.Cu") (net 1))
 (segment (start 171.495 38.05) (end 172.72 36.825) (width 0.25) (layer "B.Cu") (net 1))
 (segment (start 185.42 68.58) (end 175.26 68.58) (width 0.25) (layer "B.Cu") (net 5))
 (segment (start 177.8 27.935) (end 177.8 27.94) (width 0.25) (layer "F.Cu") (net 32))
 (segment (start 186.785 29.115) (end 178.98 29.115) (width 0.25) (layer "B.Cu") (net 32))
 (segment (start 178.98 29.115) (end 177.8 27.935) (width 0.25) (layer "B.Cu") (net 32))
 (segment (start 187.96 27.94) (end 186.785 29.115) (width 0.25) (layer "B.Cu") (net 32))
 (segment (start 184.19 26.71) (end 185.42 27.94) (width 0.25) (layer "B.Cu") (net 33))
 (segment (start 175.215 26.71) (end 184.19 26.71) (width 0.25) (layer "B.Cu") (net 33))
 (segment (start 172.72 29.205) (end 175.215 26.71) (width 0.25) (layer "B.Cu") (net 33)))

